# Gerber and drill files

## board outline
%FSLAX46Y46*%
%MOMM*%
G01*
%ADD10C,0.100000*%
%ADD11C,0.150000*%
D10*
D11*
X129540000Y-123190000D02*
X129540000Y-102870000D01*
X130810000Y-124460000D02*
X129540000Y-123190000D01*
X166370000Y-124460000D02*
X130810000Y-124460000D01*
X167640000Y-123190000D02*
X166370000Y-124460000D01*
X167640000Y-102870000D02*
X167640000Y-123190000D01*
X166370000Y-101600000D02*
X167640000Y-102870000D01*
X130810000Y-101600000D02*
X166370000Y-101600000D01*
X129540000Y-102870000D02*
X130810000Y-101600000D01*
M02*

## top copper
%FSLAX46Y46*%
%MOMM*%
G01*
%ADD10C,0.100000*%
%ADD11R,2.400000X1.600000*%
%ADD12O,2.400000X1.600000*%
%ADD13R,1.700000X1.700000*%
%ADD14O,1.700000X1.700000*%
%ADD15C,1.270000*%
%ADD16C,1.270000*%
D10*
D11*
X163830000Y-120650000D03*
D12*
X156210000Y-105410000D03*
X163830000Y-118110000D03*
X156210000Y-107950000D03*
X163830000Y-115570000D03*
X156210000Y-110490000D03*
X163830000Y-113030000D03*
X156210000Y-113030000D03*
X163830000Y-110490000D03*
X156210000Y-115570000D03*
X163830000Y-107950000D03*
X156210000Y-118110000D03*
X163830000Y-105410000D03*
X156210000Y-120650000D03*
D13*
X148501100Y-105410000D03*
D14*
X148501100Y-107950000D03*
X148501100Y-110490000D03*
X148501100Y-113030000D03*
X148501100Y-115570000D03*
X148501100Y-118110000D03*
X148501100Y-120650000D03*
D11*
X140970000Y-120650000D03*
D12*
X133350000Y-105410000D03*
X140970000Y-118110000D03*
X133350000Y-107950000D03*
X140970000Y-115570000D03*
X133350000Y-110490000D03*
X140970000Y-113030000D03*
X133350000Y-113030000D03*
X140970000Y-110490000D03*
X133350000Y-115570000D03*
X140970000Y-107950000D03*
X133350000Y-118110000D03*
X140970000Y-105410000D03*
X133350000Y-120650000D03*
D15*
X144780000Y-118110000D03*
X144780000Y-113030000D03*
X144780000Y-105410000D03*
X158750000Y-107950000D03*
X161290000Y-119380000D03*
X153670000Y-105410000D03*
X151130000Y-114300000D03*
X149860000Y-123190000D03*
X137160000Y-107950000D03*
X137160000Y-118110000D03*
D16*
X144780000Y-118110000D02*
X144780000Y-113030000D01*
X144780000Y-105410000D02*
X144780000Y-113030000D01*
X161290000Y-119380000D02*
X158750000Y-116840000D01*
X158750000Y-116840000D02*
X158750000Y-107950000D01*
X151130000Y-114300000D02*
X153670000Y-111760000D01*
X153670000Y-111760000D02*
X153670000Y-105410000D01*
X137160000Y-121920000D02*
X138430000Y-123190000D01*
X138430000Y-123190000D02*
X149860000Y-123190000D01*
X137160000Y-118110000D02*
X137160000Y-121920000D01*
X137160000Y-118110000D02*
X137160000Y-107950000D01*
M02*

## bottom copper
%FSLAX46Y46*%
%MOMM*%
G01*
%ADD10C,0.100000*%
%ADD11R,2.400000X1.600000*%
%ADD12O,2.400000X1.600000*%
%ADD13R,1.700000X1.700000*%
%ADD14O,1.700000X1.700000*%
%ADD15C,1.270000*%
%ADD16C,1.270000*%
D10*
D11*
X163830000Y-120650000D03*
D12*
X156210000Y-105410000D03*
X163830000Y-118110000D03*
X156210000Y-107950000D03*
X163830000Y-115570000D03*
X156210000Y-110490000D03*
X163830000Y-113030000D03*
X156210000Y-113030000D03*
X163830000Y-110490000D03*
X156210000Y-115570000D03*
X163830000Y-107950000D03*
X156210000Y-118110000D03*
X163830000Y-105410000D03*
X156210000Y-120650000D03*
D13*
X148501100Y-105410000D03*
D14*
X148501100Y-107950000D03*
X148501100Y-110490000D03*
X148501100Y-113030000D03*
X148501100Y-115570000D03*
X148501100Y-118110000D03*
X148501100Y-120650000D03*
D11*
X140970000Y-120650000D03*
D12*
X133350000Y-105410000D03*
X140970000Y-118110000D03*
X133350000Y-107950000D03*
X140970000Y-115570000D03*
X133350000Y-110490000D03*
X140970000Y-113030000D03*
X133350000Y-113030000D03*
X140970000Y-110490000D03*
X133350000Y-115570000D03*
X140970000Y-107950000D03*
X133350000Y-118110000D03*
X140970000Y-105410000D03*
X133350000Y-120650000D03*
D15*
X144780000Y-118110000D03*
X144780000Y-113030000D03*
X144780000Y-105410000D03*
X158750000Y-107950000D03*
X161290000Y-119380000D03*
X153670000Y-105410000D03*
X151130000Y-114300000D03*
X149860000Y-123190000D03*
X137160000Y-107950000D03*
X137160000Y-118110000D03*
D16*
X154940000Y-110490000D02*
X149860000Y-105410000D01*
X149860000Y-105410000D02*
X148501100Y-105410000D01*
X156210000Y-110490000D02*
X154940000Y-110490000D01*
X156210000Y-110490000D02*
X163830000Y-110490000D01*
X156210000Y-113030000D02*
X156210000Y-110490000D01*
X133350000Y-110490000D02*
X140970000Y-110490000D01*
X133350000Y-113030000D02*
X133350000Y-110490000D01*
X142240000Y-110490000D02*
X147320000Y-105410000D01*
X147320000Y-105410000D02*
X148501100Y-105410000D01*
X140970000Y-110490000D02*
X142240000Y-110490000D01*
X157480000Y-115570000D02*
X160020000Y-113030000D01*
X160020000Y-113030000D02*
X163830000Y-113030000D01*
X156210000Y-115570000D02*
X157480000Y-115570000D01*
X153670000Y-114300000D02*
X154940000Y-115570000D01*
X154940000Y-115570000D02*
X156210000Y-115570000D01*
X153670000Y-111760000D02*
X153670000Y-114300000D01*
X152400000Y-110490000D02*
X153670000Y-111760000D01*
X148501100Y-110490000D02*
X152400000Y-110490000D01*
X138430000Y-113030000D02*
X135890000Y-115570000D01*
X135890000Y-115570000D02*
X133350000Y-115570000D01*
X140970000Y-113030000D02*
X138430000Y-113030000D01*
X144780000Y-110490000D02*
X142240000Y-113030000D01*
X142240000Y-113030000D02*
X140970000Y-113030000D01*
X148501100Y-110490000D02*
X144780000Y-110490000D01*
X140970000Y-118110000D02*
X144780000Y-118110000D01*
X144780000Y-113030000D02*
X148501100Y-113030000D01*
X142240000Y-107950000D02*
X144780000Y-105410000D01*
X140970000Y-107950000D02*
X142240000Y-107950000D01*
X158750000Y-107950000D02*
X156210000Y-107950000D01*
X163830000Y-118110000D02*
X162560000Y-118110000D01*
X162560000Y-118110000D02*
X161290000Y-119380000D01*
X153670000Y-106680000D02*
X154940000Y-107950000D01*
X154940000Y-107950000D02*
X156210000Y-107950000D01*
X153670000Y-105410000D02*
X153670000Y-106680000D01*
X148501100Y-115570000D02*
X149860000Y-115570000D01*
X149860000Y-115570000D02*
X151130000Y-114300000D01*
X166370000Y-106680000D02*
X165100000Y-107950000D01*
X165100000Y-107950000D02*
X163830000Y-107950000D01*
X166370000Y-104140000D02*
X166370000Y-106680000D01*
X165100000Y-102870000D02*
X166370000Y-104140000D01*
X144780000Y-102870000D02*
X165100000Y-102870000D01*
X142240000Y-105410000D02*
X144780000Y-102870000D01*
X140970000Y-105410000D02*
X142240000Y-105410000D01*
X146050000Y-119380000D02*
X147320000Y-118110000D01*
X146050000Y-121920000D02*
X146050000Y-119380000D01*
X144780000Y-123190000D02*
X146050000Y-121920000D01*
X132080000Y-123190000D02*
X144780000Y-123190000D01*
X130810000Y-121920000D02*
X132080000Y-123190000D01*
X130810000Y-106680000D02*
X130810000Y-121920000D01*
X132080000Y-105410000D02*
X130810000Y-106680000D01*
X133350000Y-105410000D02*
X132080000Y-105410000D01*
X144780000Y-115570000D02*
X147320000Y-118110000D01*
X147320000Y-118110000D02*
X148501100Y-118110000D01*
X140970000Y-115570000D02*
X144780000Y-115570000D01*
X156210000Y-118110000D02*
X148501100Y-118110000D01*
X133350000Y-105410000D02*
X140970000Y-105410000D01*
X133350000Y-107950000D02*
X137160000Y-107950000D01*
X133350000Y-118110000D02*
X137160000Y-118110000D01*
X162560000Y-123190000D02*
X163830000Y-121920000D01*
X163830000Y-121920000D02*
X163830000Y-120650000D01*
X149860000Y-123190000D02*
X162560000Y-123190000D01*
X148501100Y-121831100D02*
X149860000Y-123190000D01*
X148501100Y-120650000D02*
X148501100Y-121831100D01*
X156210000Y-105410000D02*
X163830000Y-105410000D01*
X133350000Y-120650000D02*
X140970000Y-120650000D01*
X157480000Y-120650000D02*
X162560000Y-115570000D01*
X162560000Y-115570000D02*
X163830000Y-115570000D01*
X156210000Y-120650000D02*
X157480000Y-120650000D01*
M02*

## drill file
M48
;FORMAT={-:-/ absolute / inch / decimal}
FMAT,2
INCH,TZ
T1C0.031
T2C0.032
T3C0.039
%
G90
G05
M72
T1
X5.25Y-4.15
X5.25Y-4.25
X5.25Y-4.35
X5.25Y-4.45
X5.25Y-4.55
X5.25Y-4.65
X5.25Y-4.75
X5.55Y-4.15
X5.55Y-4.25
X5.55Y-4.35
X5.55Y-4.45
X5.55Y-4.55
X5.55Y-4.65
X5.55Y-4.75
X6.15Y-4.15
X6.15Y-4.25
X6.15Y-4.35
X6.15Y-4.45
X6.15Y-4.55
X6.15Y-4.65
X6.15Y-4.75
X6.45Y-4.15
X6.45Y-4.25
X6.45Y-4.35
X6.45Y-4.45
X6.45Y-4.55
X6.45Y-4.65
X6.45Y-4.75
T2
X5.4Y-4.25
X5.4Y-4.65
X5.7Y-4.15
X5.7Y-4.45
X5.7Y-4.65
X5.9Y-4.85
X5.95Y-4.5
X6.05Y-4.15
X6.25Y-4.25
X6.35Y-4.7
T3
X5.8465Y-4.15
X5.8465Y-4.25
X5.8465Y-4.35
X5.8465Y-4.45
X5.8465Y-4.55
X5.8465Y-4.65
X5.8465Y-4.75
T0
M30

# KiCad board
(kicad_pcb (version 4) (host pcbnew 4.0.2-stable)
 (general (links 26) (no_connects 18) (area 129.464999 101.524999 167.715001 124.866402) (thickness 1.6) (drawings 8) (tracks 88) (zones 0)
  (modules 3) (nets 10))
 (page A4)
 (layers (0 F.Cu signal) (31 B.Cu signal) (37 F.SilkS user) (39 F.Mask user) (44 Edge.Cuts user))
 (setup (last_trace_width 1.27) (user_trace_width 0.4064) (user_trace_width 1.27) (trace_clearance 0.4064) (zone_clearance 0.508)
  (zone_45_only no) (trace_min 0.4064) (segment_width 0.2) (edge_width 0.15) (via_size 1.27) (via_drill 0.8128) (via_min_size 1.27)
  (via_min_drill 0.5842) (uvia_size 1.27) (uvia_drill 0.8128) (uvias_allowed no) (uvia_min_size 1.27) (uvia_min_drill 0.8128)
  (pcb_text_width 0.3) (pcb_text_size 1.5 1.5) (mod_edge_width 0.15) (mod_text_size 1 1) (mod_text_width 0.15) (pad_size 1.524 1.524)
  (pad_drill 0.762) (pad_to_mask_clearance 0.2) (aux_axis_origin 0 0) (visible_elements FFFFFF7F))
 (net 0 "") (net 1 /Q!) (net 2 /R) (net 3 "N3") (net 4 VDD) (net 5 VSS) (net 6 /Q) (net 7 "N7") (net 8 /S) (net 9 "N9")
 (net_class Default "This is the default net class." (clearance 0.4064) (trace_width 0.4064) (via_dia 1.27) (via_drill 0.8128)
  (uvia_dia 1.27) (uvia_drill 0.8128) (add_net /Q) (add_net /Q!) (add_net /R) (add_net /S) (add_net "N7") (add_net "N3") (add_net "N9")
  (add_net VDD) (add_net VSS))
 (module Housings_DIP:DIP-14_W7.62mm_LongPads (layer F.Cu) (at 163.83 120.65 180)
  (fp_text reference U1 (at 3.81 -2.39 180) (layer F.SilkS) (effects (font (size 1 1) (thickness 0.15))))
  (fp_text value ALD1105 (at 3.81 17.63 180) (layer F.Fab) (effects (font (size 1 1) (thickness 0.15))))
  (pad 1 thru_hole rect (at 0 0 180) (size 2.4 1.6) (drill 0.8) (layers *.Cu *.Mask) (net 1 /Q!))
  (pad 8 thru_hole oval (at 7.62 15.24 180) (size 2.4 1.6) (drill 0.8) (layers *.Cu *.Mask) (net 1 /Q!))
  (pad 2 thru_hole oval (at 0 2.54 180) (size 2.4 1.6) (drill 0.8) (layers *.Cu *.Mask) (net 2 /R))
  (pad 9 thru_hole oval (at 7.62 12.7 180) (size 2.4 1.6) (drill 0.8) (layers *.Cu *.Mask) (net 2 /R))
  (pad 3 thru_hole oval (at 0 5.08 180) (size 2.4 1.6) (drill 0.8) (layers *.Cu *.Mask) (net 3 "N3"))
  (pad 10 thru_hole oval (at 7.62 10.16 180) (size 2.4 1.6) (drill 0.8) (layers *.Cu *.Mask) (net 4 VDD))
  (pad 4 thru_hole oval (at 0 7.62 180) (size 2.4 1.6) (drill 0.8) (layers *.Cu *.Mask) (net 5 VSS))
  (pad 11 thru_hole oval (at 7.62 7.62 180) (size 2.4 1.6) (drill 0.8) (layers *.Cu *.Mask) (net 4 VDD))
  (pad 5 thru_hole oval (at 0 10.16 180) (size 2.4 1.6) (drill 0.8) (layers *.Cu *.Mask) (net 4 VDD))
  (pad 12 thru_hole oval (at 7.62 5.08 180) (size 2.4 1.6) (drill 0.8) (layers *.Cu *.Mask) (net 5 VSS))
  (pad 6 thru_hole oval (at 0 12.7 180) (size 2.4 1.6) (drill 0.8) (layers *.Cu *.Mask) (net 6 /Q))
  (pad 13 thru_hole oval (at 7.62 2.54 180) (size 2.4 1.6) (drill 0.8) (layers *.Cu *.Mask) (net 6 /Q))
  (pad 7 thru_hole oval (at 0 15.24 180) (size 2.4 1.6) (drill 0.8) (layers *.Cu *.Mask) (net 1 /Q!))
  (pad 14 thru_hole oval (at 7.62 0 180) (size 2.4 1.6) (drill 0.8) (layers *.Cu *.Mask) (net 3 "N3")))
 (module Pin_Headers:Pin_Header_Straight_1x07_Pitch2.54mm (layer F.Cu) (at 148.5011 105.41)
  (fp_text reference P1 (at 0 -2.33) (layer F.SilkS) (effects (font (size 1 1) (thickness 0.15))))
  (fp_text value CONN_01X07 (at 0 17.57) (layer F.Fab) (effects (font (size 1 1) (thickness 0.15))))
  (pad 1 thru_hole rect (at 0 0) (size 1.7 1.7) (drill 1) (layers *.Cu *.Mask) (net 4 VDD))
  (pad 2 thru_hole oval (at 0 2.54) (size 1.7 1.7) (drill 1) (layers *.Cu *.Mask) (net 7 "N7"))
  (pad 3 thru_hole oval (at 0 5.08) (size 1.7 1.7) (drill 1) (layers *.Cu *.Mask) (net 5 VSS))
  (pad 4 thru_hole oval (at 0 7.62) (size 1.7 1.7) (drill 1) (layers *.Cu *.Mask) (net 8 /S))
  (pad 5 thru_hole oval (at 0 10.16) (size 1.7 1.7) (drill 1) (layers *.Cu *.Mask) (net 2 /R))
  (pad 6 thru_hole oval (at 0 12.7) (size 1.7 1.7) (drill 1) (layers *.Cu *.Mask) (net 6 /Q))
  (pad 7 thru_hole oval (at 0 15.24) (size 1.7 1.7) (drill 1) (layers *.Cu *.Mask) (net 1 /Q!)))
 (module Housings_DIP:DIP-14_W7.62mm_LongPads (layer F.Cu) (at 140.97 120.65 180)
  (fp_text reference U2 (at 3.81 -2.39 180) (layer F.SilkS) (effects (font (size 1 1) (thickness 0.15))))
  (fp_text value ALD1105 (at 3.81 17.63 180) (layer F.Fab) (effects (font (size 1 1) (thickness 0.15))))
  (pad 1 thru_hole rect (at 0 0 180) (size 2.4 1.6) (drill 0.8) (layers *.Cu *.Mask) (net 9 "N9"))
  (pad 8 thru_hole oval (at 7.62 15.24 180) (size 2.4 1.6) (drill 0.8) (layers *.Cu *.Mask) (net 6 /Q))
  (pad 2 thru_hole oval (at 0 2.54 180) (size 2.4 1.6) (drill 0.8) (layers *.Cu *.Mask) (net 8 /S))
  (pad 9 thru_hole oval (at 7.62 12.7 180) (size 2.4 1.6) (drill 0.8) (layers *.Cu *.Mask) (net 1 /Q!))
  (pad 3 thru_hole oval (at 0 5.08 180) (size 2.4 1.6) (drill 0.8) (layers *.Cu *.Mask) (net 6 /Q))
  (pad 10 thru_hole oval (at 7.62 10.16 180) (size 2.4 1.6) (drill 0.8) (layers *.Cu *.Mask) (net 4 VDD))
  (pad 4 thru_hole oval (at 0 7.62 180) (size 2.4 1.6) (drill 0.8) (layers *.Cu *.Mask) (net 5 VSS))
  (pad 11 thru_hole oval (at 7.62 7.62 180) (size 2.4 1.6) (drill 0.8) (layers *.Cu *.Mask) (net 4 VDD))
  (pad 5 thru_hole oval (at 0 10.16 180) (size 2.4 1.6) (drill 0.8) (layers *.Cu *.Mask) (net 4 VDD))
  (pad 12 thru_hole oval (at 7.62 5.08 180) (size 2.4 1.6) (drill 0.8) (layers *.Cu *.Mask) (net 5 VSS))
  (pad 6 thru_hole oval (at 0 12.7 180) (size 2.4 1.6) (drill 0.8) (layers *.Cu *.Mask) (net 8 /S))
  (pad 13 thru_hole oval (at 7.62 2.54 180) (size 2.4 1.6) (drill 0.8) (layers *.Cu *.Mask) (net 1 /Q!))
  (pad 7 thru_hole oval (at 0 15.24 180) (size 2.4 1.6) (drill 0.8) (layers *.Cu *.Mask) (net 6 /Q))
  (pad 14 thru_hole oval (at 7.62 0 180) (size 2.4 1.6) (drill 0.8) (layers *.Cu *.Mask) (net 9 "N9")))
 (gr_line (start 129.54 123.19) (end 129.54 102.87) (layer Edge.Cuts) (width 0.15))
 (gr_line (start 130.81 124.46) (end 129.54 123.19) (layer Edge.Cuts) (width 0.15))
 (gr_line (start 166.37 124.46) (end 130.81 124.46) (layer Edge.Cuts) (width 0.15))
 (gr_line (start 167.64 123.19) (end 166.37 124.46) (layer Edge.Cuts) (width 0.15))
 (gr_line (start 167.64 102.87) (end 167.64 123.19) (layer Edge.Cuts) (width 0.15))
 (gr_line (start 166.37 101.6) (end 167.64 102.87) (layer Edge.Cuts) (width 0.15))
 (gr_line (start 130.81 101.6) (end 166.37 101.6) (layer Edge.Cuts) (width 0.15))
 (gr_line (start 129.54 102.87) (end 130.81 101.6) (layer Edge.Cuts) (width 0.15))
 (segment (start 154.94 110.49) (end 149.86 105.41) (width 1.27) (layer B.Cu) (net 4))
 (segment (start 149.86 105.41) (end 148.5011 105.41) (width 1.27) (layer B.Cu) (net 4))
 (segment (start 156.21 110.49) (end 154.94 110.49) (width 1.27) (layer B.Cu) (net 4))
 (segment (start 156.21 110.49) (end 163.83 110.49) (width 1.27) (layer B.Cu) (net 4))
 (segment (start 156.21 113.03) (end 156.21 110.49) (width 1.27) (layer B.Cu) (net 4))
 (segment (start 133.35 110.49) (end 140.97 110.49) (width 1.27) (layer B.Cu) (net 4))
 (segment (start 133.35 113.03) (end 133.35 110.49) (width 1.27) (layer B.Cu) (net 4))
 (segment (start 142.24 110.49) (end 147.32 105.41) (width 1.27) (layer B.Cu) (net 4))
 (segment (start 147.32 105.41) (end 148.5011 105.41) (width 1.27) (layer B.Cu) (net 4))
 (segment (start 140.97 110.49) (end 142.24 110.49) (width 1.27) (layer B.Cu) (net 4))
 (segment (start 157.48 115.57) (end 160.02 113.03) (width 1.27) (layer B.Cu) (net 5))
 (segment (start 160.02 113.03) (end 163.83 113.03) (width 1.27) (layer B.Cu) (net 5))
 (segment (start 156.21 115.57) (end 157.48 115.57) (width 1.27) (layer B.Cu) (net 5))
 (segment (start 153.67 114.3) (end 154.94 115.57) (width 1.27) (layer B.Cu) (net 5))
 (segment (start 154.94 115.57) (end 156.21 115.57) (width 1.27) (layer B.Cu) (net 5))
 (segment (start 153.67 111.76) (end 153.67 114.3) (width 1.27) (layer B.Cu) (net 5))
 (segment (start 152.4 110.49) (end 153.67 111.76) (width 1.27) (layer B.Cu) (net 5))
 (segment (start 148.5011 110.49) (end 152.4 110.49) (width 1.27) (layer B.Cu) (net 5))
 (segment (start 138.43 113.03) (end 135.89 115.57) (width 1.27) (layer B.Cu) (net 5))
 (segment (start 135.89 115.57) (end 133.35 115.57) (width 1.27) (layer B.Cu) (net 5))
 (segment (start 140.97 113.03) (end 138.43 113.03) (width 1.27) (layer B.Cu) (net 5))
 (segment (start 144.78 110.49) (end 142.24 113.03) (width 1.27) (layer B.Cu) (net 5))
 (segment (start 142.24 113.03) (end 140.97 113.03) (width 1.27) (layer B.Cu) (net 5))
 (segment (start 148.5011 110.49) (end 144.78 110.49) (width 1.27) (layer B.Cu) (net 5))
 (segment (start 144.78 118.11) (end 144.78 113.03) (width 1.27) (layer F.Cu) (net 8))
 (segment (start 140.97 118.11) (end 144.78 118.11) (width 1.27) (layer B.Cu) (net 8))
 (via (at 144.78 118.11) (size 1.27) (drill 0.8128) (layers F.Cu B.Cu) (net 8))
 (segment (start 144.78 113.03) (end 148.5011 113.03) (width 1.27) (layer B.Cu) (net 8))
 (segment (start 144.78 105.41) (end 144.78 113.03) (width 1.27) (layer F.Cu) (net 8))
 (via (at 144.78 113.03) (size 1.27) (drill 0.8128) (layers F.Cu B.Cu) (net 8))
 (segment (start 142.24 107.95) (end 144.78 105.41) (width 1.27) (layer B.Cu) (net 8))
 (via (at 144.78 105.41) (size 1.27) (drill 0.8128) (layers F.Cu B.Cu) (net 8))
 (segment (start 140.97 107.95) (end 142.24 107.95) (width 1.27) (layer B.Cu) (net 8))
 (segment (start 158.75 107.95) (end 156.21 107.95) (width 1.27) (layer B.Cu) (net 2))
 (segment (start 161.29 119.38) (end 158.75 116.84) (width 1.27) (layer F.Cu) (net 2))
 (segment (start 158.75 116.84) (end 158.75 107.95) (width 1.27) (layer F.Cu) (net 2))
 (via (at 158.75 107.95) (size 1.27) (drill 0.8128) (layers F.Cu B.Cu) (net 2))
 (segment (start 163.83 118.11) (end 162.56 118.11) (width 1.27) (layer B.Cu) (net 2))
 (segment (start 162.56 118.11) (end 161.29 119.38) (width 1.27) (layer B.Cu) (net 2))
 (via (at 161.29 119.38) (size 1.27) (drill 0.8128) (layers F.Cu B.Cu) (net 2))
 (segment (start 153.67 106.68) (end 154.94 107.95) (width 1.27) (layer B.Cu) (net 2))
 (segment (start 154.94 107.95) (end 156.21 107.95) (width 1.27) (layer B.Cu) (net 2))
 (segment (start 153.67 105.41) (end 153.67 106.68) (width 1.27) (layer B.Cu) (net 2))
 (segment (start 151.13 114.3) (end 153.67 111.76) (width 1.27) (layer F.Cu) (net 2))
 (segment (start 153.67 111.76) (end 153.67 105.41) (width 1.27) (layer F.Cu) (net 2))
 (via (at 153.67 105.41) (size 1.27) (drill 0.8128) (layers F.Cu B.Cu) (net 2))
 (segment (start 148.5011 115.57) (end 149.86 115.57) (width 1.27) (layer B.Cu) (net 2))
 (segment (start 149.86 115.57) (end 151.13 114.3) (width 1.27) (layer B.Cu) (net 2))
 (via (at 151.13 114.3) (size 1.27) (drill 0.8128) (layers F.Cu B.Cu) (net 2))
 (segment (start 166.37 106.68) (end 165.1 107.95) (width 1.27) (layer B.Cu) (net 6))
 (segment (start 165.1 107.95) (end 163.83 107.95) (width 1.27) (layer B.Cu) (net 6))
 (segment (start 166.37 104.14) (end 166.37 106.68) (width 1.27) (layer B.Cu) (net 6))
 (segment (start 165.1 102.87) (end 166.37 104.14) (width 1.27) (layer B.Cu) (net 6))
 (segment (start 144.78 102.87) (end 165.1 102.87) (width 1.27) (layer B.Cu) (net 6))
 (segment (start 142.24 105.41) (end 144.78 102.87) (width 1.27) (layer B.Cu) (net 6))
 (segment (start 140.97 105.41) (end 142.24 105.41) (width 1.27) (layer B.Cu) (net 6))
 (segment (start 146.05 119.38) (end 147.32 118.11) (width 1.27) (layer B.Cu) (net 6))
 (segment (start 146.05 121.92) (end 146.05 119.38) (width 1.27) (layer B.Cu) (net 6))
 (segment (start 144.78 123.19) (end 146.05 121.92) (width 1.27) (layer B.Cu) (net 6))
 (segment (start 132.08 123.19) (end 144.78 123.19) (width 1.27) (layer B.Cu) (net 6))
 (segment (start 130.81 121.92) (end 132.08 123.19) (width 1.27) (layer B.Cu) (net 6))
 (segment (start 130.81 106.68) (end 130.81 121.92) (width 1.27) (layer B.Cu) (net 6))
 (segment (start 132.08 105.41) (end 130.81 106.68) (width 1.27) (layer B.Cu) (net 6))
 (segment (start 133.35 105.41) (end 132.08 105.41) (width 1.27) (layer B.Cu) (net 6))
 (segment (start 144.78 115.57) (end 147.32 118.11) (width 1.27) (layer B.Cu) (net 6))
 (segment (start 147.32 118.11) (end 148.5011 118.11) (width 1.27) (layer B.Cu) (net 6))
 (segment (start 140.97 115.57) (end 144.78 115.57) (width 1.27) (layer B.Cu) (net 6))
 (segment (start 156.21 118.11) (end 148.5011 118.11) (width 1.27) (layer B.Cu) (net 6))
 (segment (start 133.35 105.41) (end 140.97 105.41) (width 1.27) (layer B.Cu) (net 6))
 (segment (start 137.16 121.92) (end 138.43 123.19) (width 1.27) (layer F.Cu) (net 1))
 (segment (start 138.43 123.19) (end 149.86 123.19) (width 1.27) (layer F.Cu) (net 1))
 (via (at 149.86 123.19) (size 1.27) (drill 0.8128) (layers F.Cu B.Cu) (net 1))
 (segment (start 137.16 118.11) (end 137.16 121.92) (width 1.27) (layer F.Cu) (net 1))
 (segment (start 133.35 107.95) (end 137.16 107.95) (width 1.27) (layer B.Cu) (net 1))
 (via (at 137.16 107.95) (size 1.27) (drill 0.8128) (layers F.Cu B.Cu) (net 1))
 (segment (start 137.16 118.11) (end 137.16 107.95) (width 1.27) (layer F.Cu) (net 1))
 (segment (start 133.35 118.11) (end 137.16 118.11) (width 1.27) (layer B.Cu) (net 1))
 (via (at 137.16 118.11) (size 1.27) (drill 0.8128) (layers F.Cu B.Cu) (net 1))
 (segment (start 162.56 123.19) (end 163.83 121.92) (width 1.27) (layer B.Cu) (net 1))
 (segment (start 163.83 121.92) (end 163.83 120.65) (width 1.27) (layer B.Cu) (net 1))
 (segment (start 149.86 123.19) (end 162.56 123.19) (width 1.27) (layer B.Cu) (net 1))
 (segment (start 148.5011 121.8311) (end 149.86 123.19) (width 1.27) (layer B.Cu) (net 1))
 (segment (start 148.5011 120.65) (end 148.5011 121.8311) (width 1.27) (layer B.Cu) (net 1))
 (segment (start 156.21 105.41) (end 163.83 105.41) (width 1.27) (layer B.Cu) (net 1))
 (segment (start 133.35 120.65) (end 140.97 120.65) (width 1.27) (layer B.Cu) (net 9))
 (segment (start 157.48 120.65) (end 162.56 115.57) (width 1.27) (layer B.Cu) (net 3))
 (segment (start 162.56 115.57) (end 163.83 115.57) (width 1.27) (layer B.Cu) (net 3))
 (segment (start 156.21 120.65) (end 157.48 120.65) (width 1.27) (layer B.Cu) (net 3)))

